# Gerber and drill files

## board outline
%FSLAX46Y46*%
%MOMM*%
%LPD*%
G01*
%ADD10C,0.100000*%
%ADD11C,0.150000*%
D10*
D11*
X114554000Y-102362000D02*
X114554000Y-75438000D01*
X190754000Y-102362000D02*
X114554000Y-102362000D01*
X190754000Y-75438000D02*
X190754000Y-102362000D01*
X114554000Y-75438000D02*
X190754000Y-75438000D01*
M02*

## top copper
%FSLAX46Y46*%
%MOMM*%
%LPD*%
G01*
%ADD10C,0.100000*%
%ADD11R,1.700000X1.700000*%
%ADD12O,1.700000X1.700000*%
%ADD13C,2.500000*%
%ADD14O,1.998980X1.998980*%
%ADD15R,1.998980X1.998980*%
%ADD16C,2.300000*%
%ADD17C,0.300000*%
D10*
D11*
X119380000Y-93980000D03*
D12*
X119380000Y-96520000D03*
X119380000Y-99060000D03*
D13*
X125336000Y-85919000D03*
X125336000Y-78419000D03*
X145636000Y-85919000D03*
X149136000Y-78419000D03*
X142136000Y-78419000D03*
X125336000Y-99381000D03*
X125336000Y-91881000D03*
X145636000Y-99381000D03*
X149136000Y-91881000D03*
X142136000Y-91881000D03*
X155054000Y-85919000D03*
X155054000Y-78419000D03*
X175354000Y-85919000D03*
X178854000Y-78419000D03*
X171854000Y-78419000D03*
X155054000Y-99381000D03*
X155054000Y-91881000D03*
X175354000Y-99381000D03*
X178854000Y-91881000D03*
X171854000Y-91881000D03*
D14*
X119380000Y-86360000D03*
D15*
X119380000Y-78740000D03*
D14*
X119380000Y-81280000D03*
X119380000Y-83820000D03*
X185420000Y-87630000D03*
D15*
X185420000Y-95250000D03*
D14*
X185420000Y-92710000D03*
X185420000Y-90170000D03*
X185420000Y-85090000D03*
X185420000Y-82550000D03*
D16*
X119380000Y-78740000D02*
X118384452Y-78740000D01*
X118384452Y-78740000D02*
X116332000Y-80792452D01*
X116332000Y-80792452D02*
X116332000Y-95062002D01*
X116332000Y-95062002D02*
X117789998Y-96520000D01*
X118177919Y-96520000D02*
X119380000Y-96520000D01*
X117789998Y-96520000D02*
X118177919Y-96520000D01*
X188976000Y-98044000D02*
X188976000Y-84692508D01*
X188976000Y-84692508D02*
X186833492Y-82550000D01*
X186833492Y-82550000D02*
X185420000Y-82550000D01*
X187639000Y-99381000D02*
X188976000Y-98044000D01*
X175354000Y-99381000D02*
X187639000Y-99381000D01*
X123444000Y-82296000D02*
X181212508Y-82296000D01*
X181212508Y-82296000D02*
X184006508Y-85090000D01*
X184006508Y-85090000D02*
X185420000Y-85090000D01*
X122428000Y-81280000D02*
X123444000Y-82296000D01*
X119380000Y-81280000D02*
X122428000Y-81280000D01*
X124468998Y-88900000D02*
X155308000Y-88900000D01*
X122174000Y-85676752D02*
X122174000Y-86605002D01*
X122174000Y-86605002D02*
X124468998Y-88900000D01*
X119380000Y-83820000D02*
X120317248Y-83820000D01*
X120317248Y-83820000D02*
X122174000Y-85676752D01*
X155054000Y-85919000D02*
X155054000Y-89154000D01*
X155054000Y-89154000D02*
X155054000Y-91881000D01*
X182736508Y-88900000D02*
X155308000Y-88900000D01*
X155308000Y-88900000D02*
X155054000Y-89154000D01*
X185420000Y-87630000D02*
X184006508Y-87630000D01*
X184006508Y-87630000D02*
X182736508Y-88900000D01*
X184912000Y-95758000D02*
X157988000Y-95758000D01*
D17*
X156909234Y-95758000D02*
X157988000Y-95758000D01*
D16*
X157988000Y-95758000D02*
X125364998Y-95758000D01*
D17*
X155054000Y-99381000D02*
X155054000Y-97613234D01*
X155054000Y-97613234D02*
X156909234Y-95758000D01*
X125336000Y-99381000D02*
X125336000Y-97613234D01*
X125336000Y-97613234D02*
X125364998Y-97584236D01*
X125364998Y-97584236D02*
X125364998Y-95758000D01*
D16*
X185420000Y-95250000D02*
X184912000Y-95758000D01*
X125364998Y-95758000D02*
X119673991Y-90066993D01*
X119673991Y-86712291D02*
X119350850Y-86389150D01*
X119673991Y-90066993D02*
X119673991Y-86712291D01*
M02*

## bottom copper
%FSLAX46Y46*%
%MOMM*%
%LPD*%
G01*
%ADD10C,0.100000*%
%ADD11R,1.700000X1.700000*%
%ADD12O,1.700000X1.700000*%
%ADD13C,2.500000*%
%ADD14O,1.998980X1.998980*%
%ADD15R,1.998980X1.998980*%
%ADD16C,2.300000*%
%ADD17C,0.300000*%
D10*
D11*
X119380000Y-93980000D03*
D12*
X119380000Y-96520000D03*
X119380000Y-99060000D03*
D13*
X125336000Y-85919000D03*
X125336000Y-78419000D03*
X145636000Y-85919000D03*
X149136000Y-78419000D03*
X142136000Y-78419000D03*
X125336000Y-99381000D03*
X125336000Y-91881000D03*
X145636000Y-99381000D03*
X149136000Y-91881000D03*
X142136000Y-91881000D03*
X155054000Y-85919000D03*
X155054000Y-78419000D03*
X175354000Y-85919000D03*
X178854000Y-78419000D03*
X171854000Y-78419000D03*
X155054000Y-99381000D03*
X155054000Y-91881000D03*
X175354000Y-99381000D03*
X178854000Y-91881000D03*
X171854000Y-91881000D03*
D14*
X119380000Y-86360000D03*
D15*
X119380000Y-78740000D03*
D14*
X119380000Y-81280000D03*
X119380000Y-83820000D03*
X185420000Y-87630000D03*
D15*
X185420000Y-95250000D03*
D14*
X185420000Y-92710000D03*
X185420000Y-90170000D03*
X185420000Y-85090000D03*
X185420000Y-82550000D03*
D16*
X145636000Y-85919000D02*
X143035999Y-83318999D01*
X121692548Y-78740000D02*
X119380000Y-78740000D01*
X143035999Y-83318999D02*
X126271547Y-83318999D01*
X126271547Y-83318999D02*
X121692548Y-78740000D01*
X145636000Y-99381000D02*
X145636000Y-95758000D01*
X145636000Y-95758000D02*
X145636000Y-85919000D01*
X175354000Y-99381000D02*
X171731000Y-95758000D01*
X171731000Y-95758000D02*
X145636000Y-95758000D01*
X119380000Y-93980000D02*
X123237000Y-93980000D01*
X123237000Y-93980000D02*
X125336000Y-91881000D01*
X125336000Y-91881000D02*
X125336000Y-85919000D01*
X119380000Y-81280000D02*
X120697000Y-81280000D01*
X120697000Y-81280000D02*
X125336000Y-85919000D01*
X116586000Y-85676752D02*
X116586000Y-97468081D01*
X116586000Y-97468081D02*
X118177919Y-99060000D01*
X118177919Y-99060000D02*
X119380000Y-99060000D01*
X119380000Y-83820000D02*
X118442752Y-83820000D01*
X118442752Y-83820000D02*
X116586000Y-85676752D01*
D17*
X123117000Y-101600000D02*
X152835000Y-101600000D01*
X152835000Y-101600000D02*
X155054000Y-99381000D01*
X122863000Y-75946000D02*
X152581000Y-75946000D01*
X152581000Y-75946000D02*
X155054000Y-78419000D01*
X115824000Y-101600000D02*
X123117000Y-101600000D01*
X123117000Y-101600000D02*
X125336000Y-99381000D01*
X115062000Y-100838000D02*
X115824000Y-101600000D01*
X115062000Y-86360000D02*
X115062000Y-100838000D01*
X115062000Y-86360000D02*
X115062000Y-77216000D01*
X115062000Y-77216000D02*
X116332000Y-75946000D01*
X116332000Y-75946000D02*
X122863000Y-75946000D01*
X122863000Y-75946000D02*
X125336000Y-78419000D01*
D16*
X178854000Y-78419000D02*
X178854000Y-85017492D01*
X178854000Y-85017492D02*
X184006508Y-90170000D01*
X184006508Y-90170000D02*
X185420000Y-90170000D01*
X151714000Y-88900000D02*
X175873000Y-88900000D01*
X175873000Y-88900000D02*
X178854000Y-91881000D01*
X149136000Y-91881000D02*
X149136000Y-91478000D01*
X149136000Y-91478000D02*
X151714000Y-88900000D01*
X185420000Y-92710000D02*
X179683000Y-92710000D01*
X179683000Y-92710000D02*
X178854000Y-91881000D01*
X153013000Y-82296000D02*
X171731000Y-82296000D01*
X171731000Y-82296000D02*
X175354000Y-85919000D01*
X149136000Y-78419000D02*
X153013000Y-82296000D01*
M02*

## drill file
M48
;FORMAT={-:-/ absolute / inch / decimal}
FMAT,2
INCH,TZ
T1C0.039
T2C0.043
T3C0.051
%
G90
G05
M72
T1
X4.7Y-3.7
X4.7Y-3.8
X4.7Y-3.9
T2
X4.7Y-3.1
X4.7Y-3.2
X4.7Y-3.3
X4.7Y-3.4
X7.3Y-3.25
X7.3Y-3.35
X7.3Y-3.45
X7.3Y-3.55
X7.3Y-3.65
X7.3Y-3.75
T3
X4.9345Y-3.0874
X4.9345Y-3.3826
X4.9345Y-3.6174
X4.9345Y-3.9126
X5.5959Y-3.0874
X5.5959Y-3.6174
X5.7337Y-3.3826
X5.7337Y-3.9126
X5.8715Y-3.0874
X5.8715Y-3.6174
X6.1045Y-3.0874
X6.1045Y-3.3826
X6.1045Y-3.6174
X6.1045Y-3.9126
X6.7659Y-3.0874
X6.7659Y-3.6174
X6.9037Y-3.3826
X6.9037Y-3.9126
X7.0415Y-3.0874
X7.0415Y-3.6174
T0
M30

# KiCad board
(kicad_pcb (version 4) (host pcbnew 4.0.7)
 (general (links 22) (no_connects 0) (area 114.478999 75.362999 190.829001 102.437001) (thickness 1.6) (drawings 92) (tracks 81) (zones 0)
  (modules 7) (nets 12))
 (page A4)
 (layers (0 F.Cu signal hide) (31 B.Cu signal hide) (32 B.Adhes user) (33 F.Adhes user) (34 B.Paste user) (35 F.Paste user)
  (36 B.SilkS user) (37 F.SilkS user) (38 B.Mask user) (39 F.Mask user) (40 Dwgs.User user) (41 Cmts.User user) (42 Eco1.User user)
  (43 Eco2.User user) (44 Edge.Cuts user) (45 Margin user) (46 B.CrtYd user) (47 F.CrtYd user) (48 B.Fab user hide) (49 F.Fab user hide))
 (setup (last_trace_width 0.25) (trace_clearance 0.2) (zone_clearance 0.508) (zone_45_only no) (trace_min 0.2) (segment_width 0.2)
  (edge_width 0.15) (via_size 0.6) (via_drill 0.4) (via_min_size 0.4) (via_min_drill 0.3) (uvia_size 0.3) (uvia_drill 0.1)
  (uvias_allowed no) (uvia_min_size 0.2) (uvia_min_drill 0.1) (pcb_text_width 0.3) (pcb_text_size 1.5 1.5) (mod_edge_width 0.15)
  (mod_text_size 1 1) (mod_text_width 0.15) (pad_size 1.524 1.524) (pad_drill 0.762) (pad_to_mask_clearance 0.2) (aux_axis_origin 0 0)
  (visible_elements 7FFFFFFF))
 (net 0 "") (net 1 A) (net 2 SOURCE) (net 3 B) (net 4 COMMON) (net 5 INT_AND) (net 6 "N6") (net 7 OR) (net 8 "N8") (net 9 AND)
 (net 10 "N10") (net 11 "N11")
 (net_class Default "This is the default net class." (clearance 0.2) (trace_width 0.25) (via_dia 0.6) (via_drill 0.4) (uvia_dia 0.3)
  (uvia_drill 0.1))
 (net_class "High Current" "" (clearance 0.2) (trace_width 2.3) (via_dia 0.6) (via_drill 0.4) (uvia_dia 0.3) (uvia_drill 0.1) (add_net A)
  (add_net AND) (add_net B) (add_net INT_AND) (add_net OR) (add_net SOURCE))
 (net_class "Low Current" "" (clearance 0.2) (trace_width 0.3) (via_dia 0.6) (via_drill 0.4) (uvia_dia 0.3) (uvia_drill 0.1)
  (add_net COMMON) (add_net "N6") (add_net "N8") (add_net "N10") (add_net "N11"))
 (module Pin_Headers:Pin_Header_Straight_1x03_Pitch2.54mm (layer F.Cu) (at 119.38 93.98)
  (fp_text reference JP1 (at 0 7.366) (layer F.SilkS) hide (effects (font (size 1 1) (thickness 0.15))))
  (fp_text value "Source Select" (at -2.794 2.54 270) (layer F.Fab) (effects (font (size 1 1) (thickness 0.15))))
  (pad 1 thru_hole rect (at 0 0) (size 1.7 1.7) (drill 1) (layers *.Cu *.Mask) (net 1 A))
  (pad 2 thru_hole oval (at 0 2.54) (size 1.7 1.7) (drill 1) (layers *.Cu *.Mask) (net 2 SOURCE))
  (pad 3 thru_hole oval (at 0 5.08) (size 1.7 1.7) (drill 1) (layers *.Cu *.Mask) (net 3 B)))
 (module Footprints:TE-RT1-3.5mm (layer F.Cu) (at 135.636 82.169)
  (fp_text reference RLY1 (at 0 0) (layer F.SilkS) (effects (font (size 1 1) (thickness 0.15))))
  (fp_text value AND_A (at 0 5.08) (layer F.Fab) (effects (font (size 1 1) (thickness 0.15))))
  (pad A2 thru_hole circle (at -10.3 3.75) (size 2.5 2.5) (drill 1.3) (layers *.Cu *.Mask) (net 1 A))
  (pad A1 thru_hole circle (at -10.3 -3.75) (size 2.5 2.5) (drill 1.3) (layers *.Cu *.Mask) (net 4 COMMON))
  (pad 11 thru_hole circle (at 10 3.75) (size 2.5 2.5) (drill 1.3) (layers *.Cu *.Mask) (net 2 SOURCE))
  (pad 14 thru_hole circle (at 13.5 -3.75) (size 2.5 2.5) (drill 1.3) (layers *.Cu *.Mask) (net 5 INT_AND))
  (pad 12 thru_hole circle (at 6.5 -3.75) (size 2.5 2.5) (drill 1.3) (layers *.Cu *.Mask) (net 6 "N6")))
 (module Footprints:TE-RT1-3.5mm (layer F.Cu) (at 135.636 95.631)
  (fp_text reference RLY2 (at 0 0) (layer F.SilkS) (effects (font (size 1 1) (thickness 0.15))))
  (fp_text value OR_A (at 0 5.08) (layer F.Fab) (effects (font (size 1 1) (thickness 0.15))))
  (pad A2 thru_hole circle (at -10.3 3.75) (size 2.5 2.5) (drill 1.3) (layers *.Cu *.Mask) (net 4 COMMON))
  (pad A1 thru_hole circle (at -10.3 -3.75) (size 2.5 2.5) (drill 1.3) (layers *.Cu *.Mask) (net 1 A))
  (pad 11 thru_hole circle (at 10 3.75) (size 2.5 2.5) (drill 1.3) (layers *.Cu *.Mask) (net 2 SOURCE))
  (pad 14 thru_hole circle (at 13.5 -3.75) (size 2.5 2.5) (drill 1.3) (layers *.Cu *.Mask) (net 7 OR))
  (pad 12 thru_hole circle (at 6.5 -3.75) (size 2.5 2.5) (drill 1.3) (layers *.Cu *.Mask) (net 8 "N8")))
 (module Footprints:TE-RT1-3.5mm (layer F.Cu) (at 165.354 82.169)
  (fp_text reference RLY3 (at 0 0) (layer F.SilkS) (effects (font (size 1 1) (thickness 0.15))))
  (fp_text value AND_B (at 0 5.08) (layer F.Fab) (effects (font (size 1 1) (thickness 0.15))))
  (pad A2 thru_hole circle (at -10.3 3.75) (size 2.5 2.5) (drill 1.3) (layers *.Cu *.Mask) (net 3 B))
  (pad A1 thru_hole circle (at -10.3 -3.75) (size 2.5 2.5) (drill 1.3) (layers *.Cu *.Mask) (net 4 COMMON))
  (pad 11 thru_hole circle (at 10 3.75) (size 2.5 2.5) (drill 1.3) (layers *.Cu *.Mask) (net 5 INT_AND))
  (pad 14 thru_hole circle (at 13.5 -3.75) (size 2.5 2.5) (drill 1.3) (layers *.Cu *.Mask) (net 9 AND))
  (pad 12 thru_hole circle (at 6.5 -3.75) (size 2.5 2.5) (drill 1.3) (layers *.Cu *.Mask) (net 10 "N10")))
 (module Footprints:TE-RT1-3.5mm (layer F.Cu) (at 165.354 95.631)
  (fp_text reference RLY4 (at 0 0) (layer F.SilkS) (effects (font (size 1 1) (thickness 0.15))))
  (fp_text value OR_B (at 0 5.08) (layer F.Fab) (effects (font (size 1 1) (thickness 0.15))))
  (pad A2 thru_hole circle (at -10.3 3.75) (size 2.5 2.5) (drill 1.3) (layers *.Cu *.Mask) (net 4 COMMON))
  (pad A1 thru_hole circle (at -10.3 -3.75) (size 2.5 2.5) (drill 1.3) (layers *.Cu *.Mask) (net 3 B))
  (pad 11 thru_hole circle (at 10 3.75) (size 2.5 2.5) (drill 1.3) (layers *.Cu *.Mask) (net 2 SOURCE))
  (pad 14 thru_hole circle (at 13.5 -3.75) (size 2.5 2.5) (drill 1.3) (layers *.Cu *.Mask) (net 7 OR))
  (pad 12 thru_hole circle (at 6.5 -3.75) (size 2.5 2.5) (drill 1.3) (layers *.Cu *.Mask) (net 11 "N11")))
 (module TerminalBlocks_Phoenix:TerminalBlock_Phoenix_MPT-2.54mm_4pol (layer F.Cu) (at 119.38 78.74 270)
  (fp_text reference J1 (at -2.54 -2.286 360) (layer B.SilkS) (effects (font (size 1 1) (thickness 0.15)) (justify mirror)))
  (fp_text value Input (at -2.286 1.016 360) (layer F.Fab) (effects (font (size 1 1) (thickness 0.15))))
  (pad 4 thru_hole oval (at 7.62 0 90) (size 1.99898 1.99898) (drill 1.09728) (layers *.Cu *.Mask) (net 4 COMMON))
  (pad 1 thru_hole rect (at 0 0 90) (size 1.99898 1.99898) (drill 1.09728) (layers *.Cu *.Mask) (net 2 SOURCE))
  (pad 2 thru_hole oval (at 2.54 0 90) (size 1.99898 1.99898) (drill 1.09728) (layers *.Cu *.Mask) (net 1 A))
  (pad 3 thru_hole oval (at 5.08 0 90) (size 1.99898 1.99898) (drill 1.09728) (layers *.Cu *.Mask) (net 3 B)))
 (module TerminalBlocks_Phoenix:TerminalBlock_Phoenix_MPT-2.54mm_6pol (layer F.Cu) (at 185.42 95.25 90)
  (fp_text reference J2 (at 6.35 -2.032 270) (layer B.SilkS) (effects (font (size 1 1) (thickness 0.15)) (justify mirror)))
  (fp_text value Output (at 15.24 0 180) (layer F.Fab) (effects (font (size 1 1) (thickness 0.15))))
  (pad 4 thru_hole oval (at 7.62 0 270) (size 1.99898 1.99898) (drill 1.09728) (layers *.Cu *.Mask) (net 3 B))
  (pad 1 thru_hole rect (at 0 0 270) (size 1.99898 1.99898) (drill 1.09728) (layers *.Cu *.Mask) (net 4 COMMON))
  (pad 2 thru_hole oval (at 2.54 0 270) (size 1.99898 1.99898) (drill 1.09728) (layers *.Cu *.Mask) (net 7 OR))
  (pad 3 thru_hole oval (at 5.08 0 270) (size 1.99898 1.99898) (drill 1.09728) (layers *.Cu *.Mask) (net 9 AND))
  (pad 5 thru_hole oval (at 10.16 0 270) (size 1.99898 1.99898) (drill 1.09728) (layers *.Cu *.Mask) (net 1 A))
  (pad 6 thru_hole oval (at 12.7 0 270) (size 1.99898 1.99898) (drill 1.09728) (layers *.Cu *.Mask) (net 2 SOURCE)))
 (gr_line (start 114.554 102.362) (end 114.554 75.438) (layer Edge.Cuts) (width 0.15))
 (gr_line (start 190.754 102.362) (end 114.554 102.362) (layer Edge.Cuts) (width 0.15))
 (gr_line (start 190.754 75.438) (end 190.754 102.362) (layer Edge.Cuts) (width 0.15))
 (gr_line (start 114.554 75.438) (end 190.754 75.438) (layer Edge.Cuts) (width 0.15))
 (segment (start 119.38 78.74) (end 118.384452 78.74) (width 2.3) (layer F.Cu) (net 2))
 (segment (start 118.384452 78.74) (end 116.332 80.792452) (width 2.3) (layer F.Cu) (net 2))
 (segment (start 116.332 80.792452) (end 116.332 95.062002) (width 2.3) (layer F.Cu) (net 2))
 (segment (start 116.332 95.062002) (end 117.789998 96.52) (width 2.3) (layer F.Cu) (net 2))
 (segment (start 118.177919 96.52) (end 119.38 96.52) (width 2.3) (layer F.Cu) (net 2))
 (segment (start 117.789998 96.52) (end 118.177919 96.52) (width 2.3) (layer F.Cu) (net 2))
 (segment (start 145.636 85.919) (end 143.035999 83.318999) (width 2.3) (layer B.Cu) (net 2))
 (segment (start 121.692548 78.74) (end 119.38 78.74) (width 2.3) (layer B.Cu) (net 2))
 (segment (start 143.035999 83.318999) (end 126.271547 83.318999) (width 2.3) (layer B.Cu) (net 2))
 (segment (start 126.271547 83.318999) (end 121.692548 78.74) (width 2.3) (layer B.Cu) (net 2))
 (segment (start 188.976 98.044) (end 188.976 84.692508) (width 2.3) (layer F.Cu) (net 2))
 (segment (start 188.976 84.692508) (end 186.833492 82.55) (width 2.3) (layer F.Cu) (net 2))
 (segment (start 186.833492 82.55) (end 185.42 82.55) (width 2.3) (layer F.Cu) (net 2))
 (segment (start 187.639 99.381) (end 188.976 98.044) (width 2.3) (layer F.Cu) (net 2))
 (segment (start 175.354 99.381) (end 187.639 99.381) (width 2.3) (layer F.Cu) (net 2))
 (segment (start 145.636 99.381) (end 145.636 95.758) (width 2.3) (layer B.Cu) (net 2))
 (segment (start 145.636 95.758) (end 145.636 85.919) (width 2.3) (layer B.Cu) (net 2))
 (segment (start 175.354 99.381) (end 171.731 95.758) (width 2.3) (layer B.Cu) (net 2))
 (segment (start 171.731 95.758) (end 145.636 95.758) (width 2.3) (layer B.Cu) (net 2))
 (segment (start 123.444 82.296) (end 181.212508 82.296) (width 2.3) (layer F.Cu) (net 1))
 (segment (start 181.212508 82.296) (end 184.006508 85.09) (width 2.3) (layer F.Cu) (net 1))
 (segment (start 184.006508 85.09) (end 185.42 85.09) (width 2.3) (layer F.Cu) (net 1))
 (segment (start 122.428 81.28) (end 123.444 82.296) (width 2.3) (layer F.Cu) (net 1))
 (segment (start 119.38 81.28) (end 122.428 81.28) (width 2.3) (layer F.Cu) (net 1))
 (segment (start 119.38 93.98) (end 123.237 93.98) (width 2.3) (layer B.Cu) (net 1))
 (segment (start 123.237 93.98) (end 125.336 91.881) (width 2.3) (layer B.Cu) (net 1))
 (segment (start 125.336 91.881) (end 125.336 85.919) (width 2.3) (layer B.Cu) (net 1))
 (segment (start 119.38 81.28) (end 120.697 81.28) (width 2.3) (layer B.Cu) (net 1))
 (segment (start 120.697 81.28) (end 125.336 85.919) (width 2.3) (layer B.Cu) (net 1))
 (segment (start 116.586 85.676752) (end 116.586 97.468081) (width 2.3) (layer B.Cu) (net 3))
 (segment (start 116.586 97.468081) (end 118.177919 99.06) (width 2.3) (layer B.Cu) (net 3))
 (segment (start 118.177919 99.06) (end 119.38 99.06) (width 2.3) (layer B.Cu) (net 3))
 (segment (start 119.38 83.82) (end 118.442752 83.82) (width 2.3) (layer B.Cu) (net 3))
 (segment (start 118.442752 83.82) (end 116.586 85.676752) (width 2.3) (layer B.Cu) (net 3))
 (segment (start 124.468998 88.9) (end 155.308 88.9) (width 2.3) (layer F.Cu) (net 3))
 (segment (start 122.174 85.676752) (end 122.174 86.605002) (width 2.3) (layer F.Cu) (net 3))
 (segment (start 122.174 86.605002) (end 124.468998 88.9) (width 2.3) (layer F.Cu) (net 3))
 (segment (start 119.38 83.82) (end 120.317248 83.82) (width 2.3) (layer F.Cu) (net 3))
 (segment (start 120.317248 83.82) (end 122.174 85.676752) (width 2.3) (layer F.Cu) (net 3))
 (segment (start 155.054 85.919) (end 155.054 89.154) (width 2.3) (layer F.Cu) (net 3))
 (segment (start 155.054 89.154) (end 155.054 91.881) (width 2.3) (layer F.Cu) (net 3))
 (segment (start 182.736508 88.9) (end 155.308 88.9) (width 2.3) (layer F.Cu) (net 3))
 (segment (start 155.308 88.9) (end 155.054 89.154) (width 2.3) (layer F.Cu) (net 3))
 (segment (start 185.42 87.63) (end 184.006508 87.63) (width 2.3) (layer F.Cu) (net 3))
 (segment (start 184.006508 87.63) (end 182.736508 88.9) (width 2.3) (layer F.Cu) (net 3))
 (segment (start 184.912 95.758) (end 157.988 95.758) (width 2.3) (layer F.Cu) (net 4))
 (segment (start 156.909234 95.758) (end 157.988 95.758) (width 0.3) (layer F.Cu) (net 4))
 (segment (start 157.988 95.758) (end 125.364998 95.758) (width 2.3) (layer F.Cu) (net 4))
 (segment (start 155.054 99.381) (end 155.054 97.613234) (width 0.3) (layer F.Cu) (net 4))
 (segment (start 155.054 97.613234) (end 156.909234 95.758) (width 0.3) (layer F.Cu) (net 4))
 (segment (start 125.336 99.381) (end 125.336 97.613234) (width 0.3) (layer F.Cu) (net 4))
 (segment (start 125.336 97.613234) (end 125.364998 97.584236) (width 0.3) (layer F.Cu) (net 4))
 (segment (start 125.364998 97.584236) (end 125.364998 95.758) (width 0.3) (layer F.Cu) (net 4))
 (segment (start 185.42 95.25) (end 184.912 95.758) (width 2.3) (layer F.Cu) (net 4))
 (segment (start 125.364998 95.758) (end 119.673991 90.066993) (width 2.3) (layer F.Cu) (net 4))
 (segment (start 119.673991 86.712291) (end 119.35085 86.38915) (width 2.3) (layer F.Cu) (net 4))
 (segment (start 119.673991 90.066993) (end 119.673991 86.712291) (width 2.3) (layer F.Cu) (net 4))
 (segment (start 123.117 101.6) (end 152.835 101.6) (width 0.3) (layer B.Cu) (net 4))
 (segment (start 152.835 101.6) (end 155.054 99.381) (width 0.3) (layer B.Cu) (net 4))
 (segment (start 122.863 75.946) (end 152.581 75.946) (width 0.3) (layer B.Cu) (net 4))
 (segment (start 152.581 75.946) (end 155.054 78.419) (width 0.3) (layer B.Cu) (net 4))
 (segment (start 115.824 101.6) (end 123.117 101.6) (width 0.3) (layer B.Cu) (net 4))
 (segment (start 123.117 101.6) (end 125.336 99.381) (width 0.3) (layer B.Cu) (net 4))
 (segment (start 115.062 100.838) (end 115.824 101.6) (width 0.3) (layer B.Cu) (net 4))
 (segment (start 115.062 86.36) (end 115.062 100.838) (width 0.3) (layer B.Cu) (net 4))
 (segment (start 115.062 86.36) (end 115.062 77.216) (width 0.3) (layer B.Cu) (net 4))
 (segment (start 115.062 77.216) (end 116.332 75.946) (width 0.3) (layer B.Cu) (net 4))
 (segment (start 116.332 75.946) (end 122.863 75.946) (width 0.3) (layer B.Cu) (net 4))
 (segment (start 122.863 75.946) (end 125.336 78.419) (width 0.3) (layer B.Cu) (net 4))
 (segment (start 178.854 78.419) (end 178.854 85.017492) (width 2.3) (layer B.Cu) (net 9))
 (segment (start 178.854 85.017492) (end 184.006508 90.17) (width 2.3) (layer B.Cu) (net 9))
 (segment (start 184.006508 90.17) (end 185.42 90.17) (width 2.3) (layer B.Cu) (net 9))
 (segment (start 151.714 88.9) (end 175.873 88.9) (width 2.3) (layer B.Cu) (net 7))
 (segment (start 175.873 88.9) (end 178.854 91.881) (width 2.3) (layer B.Cu) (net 7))
 (segment (start 149.136 91.881) (end 149.136 91.478) (width 2.3) (layer B.Cu) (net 7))
 (segment (start 149.136 91.478) (end 151.714 88.9) (width 2.3) (layer B.Cu) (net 7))
 (segment (start 185.42 92.71) (end 179.683 92.71) (width 2.3) (layer B.Cu) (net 7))
 (segment (start 179.683 92.71) (end 178.854 91.881) (width 2.3) (layer B.Cu) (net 7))
 (segment (start 153.013 82.296) (end 171.731 82.296) (width 2.3) (layer B.Cu) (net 5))
 (segment (start 171.731 82.296) (end 175.354 85.919) (width 2.3) (layer B.Cu) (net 5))
 (segment (start 149.136 78.419) (end 153.013 82.296) (width 2.3) (layer B.Cu) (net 5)))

